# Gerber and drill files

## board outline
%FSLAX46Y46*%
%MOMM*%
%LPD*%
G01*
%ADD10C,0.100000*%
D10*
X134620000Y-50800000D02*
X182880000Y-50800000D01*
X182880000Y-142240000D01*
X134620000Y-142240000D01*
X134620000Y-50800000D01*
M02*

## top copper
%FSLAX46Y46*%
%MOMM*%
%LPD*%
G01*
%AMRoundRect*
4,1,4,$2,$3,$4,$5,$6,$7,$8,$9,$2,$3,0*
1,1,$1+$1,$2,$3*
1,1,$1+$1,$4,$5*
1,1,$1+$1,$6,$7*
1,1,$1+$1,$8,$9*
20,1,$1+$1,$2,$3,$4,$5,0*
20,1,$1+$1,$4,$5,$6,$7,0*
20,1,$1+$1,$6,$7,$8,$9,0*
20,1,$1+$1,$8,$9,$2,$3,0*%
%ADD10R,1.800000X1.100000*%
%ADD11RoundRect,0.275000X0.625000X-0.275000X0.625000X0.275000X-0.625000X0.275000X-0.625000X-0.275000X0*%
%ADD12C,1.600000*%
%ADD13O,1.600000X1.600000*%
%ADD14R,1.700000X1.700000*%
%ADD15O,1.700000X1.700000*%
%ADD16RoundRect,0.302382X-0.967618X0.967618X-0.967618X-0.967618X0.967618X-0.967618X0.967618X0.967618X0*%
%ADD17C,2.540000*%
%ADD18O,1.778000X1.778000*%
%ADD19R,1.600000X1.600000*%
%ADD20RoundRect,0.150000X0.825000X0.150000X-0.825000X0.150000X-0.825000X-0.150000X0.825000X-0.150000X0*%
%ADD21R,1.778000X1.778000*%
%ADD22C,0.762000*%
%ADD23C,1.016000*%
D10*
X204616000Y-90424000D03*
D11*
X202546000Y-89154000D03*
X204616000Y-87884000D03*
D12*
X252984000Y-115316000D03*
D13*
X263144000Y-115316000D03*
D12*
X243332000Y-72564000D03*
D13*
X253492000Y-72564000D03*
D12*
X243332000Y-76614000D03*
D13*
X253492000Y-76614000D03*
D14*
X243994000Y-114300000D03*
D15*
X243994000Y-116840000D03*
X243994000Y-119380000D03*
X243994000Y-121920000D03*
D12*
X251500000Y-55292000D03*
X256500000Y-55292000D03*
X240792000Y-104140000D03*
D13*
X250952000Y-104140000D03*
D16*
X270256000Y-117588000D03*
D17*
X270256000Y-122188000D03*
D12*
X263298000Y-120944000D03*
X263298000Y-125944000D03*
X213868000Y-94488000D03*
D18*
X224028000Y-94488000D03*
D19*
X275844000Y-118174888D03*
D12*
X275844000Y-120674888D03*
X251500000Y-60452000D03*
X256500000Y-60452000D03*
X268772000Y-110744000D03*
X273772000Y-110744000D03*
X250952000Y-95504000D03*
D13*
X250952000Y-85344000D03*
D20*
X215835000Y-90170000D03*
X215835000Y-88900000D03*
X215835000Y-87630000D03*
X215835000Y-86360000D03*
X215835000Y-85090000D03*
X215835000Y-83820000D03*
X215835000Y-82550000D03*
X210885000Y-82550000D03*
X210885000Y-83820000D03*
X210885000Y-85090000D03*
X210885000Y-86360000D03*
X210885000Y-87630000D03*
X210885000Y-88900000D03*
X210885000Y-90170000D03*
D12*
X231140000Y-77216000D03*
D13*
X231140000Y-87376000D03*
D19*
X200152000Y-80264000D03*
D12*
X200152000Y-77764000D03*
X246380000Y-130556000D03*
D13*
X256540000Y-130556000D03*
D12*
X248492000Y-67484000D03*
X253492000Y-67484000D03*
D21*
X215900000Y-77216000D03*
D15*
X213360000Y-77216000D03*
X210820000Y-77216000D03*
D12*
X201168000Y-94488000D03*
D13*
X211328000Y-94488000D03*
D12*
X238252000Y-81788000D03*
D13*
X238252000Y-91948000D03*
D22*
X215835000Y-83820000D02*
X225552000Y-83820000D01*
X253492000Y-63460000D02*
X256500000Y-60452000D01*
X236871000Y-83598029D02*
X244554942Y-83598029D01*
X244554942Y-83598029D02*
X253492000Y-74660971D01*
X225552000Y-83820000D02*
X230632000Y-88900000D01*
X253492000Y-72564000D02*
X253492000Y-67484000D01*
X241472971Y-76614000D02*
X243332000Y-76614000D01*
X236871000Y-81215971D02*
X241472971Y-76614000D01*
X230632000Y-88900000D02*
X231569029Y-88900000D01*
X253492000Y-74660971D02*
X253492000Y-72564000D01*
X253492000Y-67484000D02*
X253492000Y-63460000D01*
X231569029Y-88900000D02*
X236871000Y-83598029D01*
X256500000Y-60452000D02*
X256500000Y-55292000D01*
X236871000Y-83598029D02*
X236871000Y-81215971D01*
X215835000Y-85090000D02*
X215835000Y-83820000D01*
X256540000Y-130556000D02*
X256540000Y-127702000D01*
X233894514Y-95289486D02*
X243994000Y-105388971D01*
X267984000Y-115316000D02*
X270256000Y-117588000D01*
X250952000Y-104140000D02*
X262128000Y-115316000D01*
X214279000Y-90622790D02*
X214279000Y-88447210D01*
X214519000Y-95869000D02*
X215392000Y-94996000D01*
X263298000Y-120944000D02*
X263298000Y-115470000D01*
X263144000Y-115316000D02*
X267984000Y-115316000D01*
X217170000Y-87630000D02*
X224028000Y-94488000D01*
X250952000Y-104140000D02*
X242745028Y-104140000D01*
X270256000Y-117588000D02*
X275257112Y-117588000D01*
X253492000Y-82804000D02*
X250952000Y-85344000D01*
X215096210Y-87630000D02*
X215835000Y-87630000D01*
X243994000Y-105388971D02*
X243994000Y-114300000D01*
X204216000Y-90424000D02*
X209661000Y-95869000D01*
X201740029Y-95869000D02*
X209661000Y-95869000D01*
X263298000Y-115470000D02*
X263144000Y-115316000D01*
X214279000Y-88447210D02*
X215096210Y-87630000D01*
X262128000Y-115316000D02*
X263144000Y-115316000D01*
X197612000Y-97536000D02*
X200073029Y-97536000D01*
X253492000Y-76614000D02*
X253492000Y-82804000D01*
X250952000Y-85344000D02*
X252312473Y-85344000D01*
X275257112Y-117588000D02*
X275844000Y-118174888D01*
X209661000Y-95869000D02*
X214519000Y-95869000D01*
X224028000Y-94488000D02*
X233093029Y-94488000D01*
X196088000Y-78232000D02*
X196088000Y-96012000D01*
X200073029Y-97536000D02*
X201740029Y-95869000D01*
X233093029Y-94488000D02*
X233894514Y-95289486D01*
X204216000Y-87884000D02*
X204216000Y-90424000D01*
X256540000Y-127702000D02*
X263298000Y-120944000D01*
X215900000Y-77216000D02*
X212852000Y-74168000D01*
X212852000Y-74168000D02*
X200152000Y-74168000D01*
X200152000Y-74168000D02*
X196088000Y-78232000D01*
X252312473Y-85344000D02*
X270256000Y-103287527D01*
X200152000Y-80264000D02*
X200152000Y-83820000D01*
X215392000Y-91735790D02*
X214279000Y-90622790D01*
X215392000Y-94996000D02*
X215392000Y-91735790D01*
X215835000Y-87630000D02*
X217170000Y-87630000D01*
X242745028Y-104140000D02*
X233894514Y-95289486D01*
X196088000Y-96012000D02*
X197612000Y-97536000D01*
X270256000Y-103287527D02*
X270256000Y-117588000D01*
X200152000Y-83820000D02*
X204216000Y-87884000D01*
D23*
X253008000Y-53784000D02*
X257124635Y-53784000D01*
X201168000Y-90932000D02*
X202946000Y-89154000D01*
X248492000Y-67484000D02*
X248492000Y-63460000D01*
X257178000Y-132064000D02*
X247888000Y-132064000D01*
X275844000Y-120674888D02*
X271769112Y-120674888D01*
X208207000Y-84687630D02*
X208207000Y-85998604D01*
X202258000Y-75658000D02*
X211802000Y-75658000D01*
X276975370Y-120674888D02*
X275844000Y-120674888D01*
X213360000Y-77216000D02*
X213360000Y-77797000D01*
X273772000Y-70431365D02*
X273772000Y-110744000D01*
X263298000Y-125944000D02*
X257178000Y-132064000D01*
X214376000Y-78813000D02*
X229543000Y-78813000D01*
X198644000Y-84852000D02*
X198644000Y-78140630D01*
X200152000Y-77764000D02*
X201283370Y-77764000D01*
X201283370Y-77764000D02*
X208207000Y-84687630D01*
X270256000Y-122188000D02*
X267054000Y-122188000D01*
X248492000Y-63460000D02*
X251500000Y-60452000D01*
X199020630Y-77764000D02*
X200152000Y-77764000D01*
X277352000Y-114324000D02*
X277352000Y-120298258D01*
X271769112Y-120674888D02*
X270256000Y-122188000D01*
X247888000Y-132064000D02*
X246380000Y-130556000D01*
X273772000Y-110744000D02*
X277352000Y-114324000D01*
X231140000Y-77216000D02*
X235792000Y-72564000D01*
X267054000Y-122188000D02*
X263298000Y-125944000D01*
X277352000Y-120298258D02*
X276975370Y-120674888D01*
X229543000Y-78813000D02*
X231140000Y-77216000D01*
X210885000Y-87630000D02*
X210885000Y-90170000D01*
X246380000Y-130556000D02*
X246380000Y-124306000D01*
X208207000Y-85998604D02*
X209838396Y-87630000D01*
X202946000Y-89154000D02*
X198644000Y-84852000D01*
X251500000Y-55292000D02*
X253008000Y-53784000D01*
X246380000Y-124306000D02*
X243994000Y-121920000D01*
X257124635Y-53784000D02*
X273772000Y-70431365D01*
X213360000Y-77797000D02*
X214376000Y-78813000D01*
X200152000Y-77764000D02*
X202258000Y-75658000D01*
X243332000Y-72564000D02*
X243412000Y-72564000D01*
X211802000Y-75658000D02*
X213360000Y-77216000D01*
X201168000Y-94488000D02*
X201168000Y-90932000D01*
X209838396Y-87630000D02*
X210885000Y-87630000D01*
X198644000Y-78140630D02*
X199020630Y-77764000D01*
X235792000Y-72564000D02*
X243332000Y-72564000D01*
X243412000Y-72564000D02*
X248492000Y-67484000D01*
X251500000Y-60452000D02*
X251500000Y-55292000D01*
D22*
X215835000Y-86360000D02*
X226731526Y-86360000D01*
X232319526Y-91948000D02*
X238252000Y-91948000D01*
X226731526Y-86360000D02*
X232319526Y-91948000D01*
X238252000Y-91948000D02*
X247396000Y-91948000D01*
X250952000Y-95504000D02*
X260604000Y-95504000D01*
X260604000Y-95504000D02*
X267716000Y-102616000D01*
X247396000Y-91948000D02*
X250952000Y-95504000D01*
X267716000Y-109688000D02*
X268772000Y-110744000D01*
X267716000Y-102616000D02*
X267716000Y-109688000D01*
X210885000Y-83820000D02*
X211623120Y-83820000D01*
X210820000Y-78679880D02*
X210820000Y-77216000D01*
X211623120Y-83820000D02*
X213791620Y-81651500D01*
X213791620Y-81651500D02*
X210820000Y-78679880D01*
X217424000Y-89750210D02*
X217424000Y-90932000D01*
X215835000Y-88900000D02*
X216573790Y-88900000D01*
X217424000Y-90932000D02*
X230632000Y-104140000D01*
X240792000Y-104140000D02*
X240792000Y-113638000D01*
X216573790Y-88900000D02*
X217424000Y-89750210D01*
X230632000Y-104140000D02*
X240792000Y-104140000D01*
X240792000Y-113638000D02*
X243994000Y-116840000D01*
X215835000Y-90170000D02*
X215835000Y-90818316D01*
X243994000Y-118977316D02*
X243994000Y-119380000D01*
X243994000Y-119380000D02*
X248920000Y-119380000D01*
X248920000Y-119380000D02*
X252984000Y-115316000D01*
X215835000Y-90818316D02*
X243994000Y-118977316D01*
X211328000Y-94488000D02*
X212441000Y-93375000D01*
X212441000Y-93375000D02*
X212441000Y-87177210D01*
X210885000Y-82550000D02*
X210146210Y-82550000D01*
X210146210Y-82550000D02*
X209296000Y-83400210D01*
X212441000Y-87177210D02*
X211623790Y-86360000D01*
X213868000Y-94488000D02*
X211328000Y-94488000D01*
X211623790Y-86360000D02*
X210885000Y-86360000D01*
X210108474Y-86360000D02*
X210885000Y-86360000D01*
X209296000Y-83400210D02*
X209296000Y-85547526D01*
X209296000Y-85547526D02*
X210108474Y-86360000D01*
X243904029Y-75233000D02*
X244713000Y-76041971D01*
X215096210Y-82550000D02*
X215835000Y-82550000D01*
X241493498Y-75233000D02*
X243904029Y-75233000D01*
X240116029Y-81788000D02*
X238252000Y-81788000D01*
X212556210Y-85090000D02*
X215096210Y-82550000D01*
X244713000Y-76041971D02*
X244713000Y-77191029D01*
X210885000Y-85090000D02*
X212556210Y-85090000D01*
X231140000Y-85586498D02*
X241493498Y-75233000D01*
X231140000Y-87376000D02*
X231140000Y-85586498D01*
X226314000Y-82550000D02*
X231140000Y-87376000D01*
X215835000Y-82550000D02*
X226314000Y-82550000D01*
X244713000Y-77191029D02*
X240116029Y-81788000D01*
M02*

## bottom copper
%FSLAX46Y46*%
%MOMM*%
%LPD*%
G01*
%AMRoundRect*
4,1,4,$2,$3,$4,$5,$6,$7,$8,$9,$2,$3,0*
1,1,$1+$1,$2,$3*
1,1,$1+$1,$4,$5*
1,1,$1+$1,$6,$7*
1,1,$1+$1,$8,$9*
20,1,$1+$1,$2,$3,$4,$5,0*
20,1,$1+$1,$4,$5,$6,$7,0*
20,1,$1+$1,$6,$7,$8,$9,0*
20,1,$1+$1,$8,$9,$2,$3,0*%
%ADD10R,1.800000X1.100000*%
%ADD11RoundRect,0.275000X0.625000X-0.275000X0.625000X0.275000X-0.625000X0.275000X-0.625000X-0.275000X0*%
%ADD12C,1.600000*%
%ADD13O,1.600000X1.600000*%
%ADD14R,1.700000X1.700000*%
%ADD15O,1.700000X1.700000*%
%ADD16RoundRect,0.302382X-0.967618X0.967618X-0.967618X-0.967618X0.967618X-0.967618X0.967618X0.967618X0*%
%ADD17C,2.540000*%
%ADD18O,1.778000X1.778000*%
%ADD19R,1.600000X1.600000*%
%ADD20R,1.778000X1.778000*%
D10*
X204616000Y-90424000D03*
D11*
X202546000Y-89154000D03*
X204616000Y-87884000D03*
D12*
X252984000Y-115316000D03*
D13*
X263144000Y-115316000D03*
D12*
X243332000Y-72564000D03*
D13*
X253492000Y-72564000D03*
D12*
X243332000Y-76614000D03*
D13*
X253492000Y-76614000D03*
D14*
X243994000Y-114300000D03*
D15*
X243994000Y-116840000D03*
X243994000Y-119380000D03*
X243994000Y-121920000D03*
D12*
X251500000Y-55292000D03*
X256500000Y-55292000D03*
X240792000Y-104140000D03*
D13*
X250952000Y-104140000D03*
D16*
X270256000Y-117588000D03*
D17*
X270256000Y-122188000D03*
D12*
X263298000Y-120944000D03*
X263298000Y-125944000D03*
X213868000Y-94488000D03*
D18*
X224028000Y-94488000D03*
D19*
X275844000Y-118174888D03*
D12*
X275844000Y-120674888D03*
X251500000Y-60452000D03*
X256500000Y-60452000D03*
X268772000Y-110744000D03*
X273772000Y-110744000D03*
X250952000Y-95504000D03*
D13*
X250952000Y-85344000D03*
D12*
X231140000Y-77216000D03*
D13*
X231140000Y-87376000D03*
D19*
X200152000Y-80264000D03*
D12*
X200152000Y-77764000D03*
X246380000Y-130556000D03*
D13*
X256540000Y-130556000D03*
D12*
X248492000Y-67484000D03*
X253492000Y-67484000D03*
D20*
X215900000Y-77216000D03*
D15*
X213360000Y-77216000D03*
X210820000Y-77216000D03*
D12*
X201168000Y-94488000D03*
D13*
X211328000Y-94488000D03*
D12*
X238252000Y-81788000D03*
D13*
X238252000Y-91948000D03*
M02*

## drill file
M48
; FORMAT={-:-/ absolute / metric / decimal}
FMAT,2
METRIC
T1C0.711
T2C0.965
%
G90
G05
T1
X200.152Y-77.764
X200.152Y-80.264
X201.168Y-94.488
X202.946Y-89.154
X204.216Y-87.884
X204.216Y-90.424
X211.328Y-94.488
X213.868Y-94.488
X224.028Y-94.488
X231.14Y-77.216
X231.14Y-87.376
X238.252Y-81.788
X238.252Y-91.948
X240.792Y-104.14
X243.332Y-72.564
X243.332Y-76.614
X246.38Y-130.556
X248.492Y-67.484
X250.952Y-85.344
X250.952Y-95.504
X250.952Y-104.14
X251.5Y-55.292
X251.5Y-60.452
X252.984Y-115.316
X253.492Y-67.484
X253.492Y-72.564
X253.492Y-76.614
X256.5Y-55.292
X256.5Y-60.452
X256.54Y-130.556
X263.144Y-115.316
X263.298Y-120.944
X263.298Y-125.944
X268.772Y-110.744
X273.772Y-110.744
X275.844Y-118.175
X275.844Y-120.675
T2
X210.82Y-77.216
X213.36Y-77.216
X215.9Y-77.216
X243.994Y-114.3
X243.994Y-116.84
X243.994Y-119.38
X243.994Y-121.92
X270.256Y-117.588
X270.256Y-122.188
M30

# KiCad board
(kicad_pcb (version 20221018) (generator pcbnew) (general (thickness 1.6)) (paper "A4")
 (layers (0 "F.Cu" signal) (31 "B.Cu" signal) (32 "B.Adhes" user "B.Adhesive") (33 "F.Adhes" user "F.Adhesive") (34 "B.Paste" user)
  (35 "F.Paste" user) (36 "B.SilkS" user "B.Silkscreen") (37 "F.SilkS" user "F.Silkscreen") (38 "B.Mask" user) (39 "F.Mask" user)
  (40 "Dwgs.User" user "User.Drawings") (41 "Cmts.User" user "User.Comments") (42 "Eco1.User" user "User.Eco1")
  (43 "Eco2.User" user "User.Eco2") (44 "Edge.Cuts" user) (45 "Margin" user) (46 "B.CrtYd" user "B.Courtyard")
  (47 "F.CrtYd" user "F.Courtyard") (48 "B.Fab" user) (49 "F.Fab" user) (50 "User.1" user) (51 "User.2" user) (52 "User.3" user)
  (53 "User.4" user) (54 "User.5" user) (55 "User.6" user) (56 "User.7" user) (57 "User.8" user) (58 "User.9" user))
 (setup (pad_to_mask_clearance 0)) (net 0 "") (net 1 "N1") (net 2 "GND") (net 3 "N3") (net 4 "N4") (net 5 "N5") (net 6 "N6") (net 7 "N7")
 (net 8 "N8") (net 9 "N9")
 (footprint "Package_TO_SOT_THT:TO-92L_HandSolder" (layer "F.Cu") (at 204.216 90.424 90)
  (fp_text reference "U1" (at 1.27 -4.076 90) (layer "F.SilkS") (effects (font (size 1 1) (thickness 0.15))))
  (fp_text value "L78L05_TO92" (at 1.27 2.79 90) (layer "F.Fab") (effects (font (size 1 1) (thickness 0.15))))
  (pad "1" thru_hole rect (at 0 0 90) (size 1.1 1.8) (drill 0.7112 (offset 0 0.4)) (layers "*.Cu" "*.Mask") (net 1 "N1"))
  (pad "2" thru_hole roundrect (at 1.27 -1.27 90) (size 1.1 1.8) (drill 0.7112 (offset 0 -0.4)) (layers "*.Cu" "*.Mask")
   (roundrect_rratio 0.25) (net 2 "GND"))
  (pad "3" thru_hole roundrect (at 2.54 0 90) (size 1.1 1.8) (drill 0.7112 (offset 0 0.4)) (layers "*.Cu" "*.Mask") (roundrect_rratio 0.25)
   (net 1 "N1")))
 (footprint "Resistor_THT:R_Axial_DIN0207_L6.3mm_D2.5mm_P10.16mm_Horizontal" (layer "F.Cu") (at 252.984 115.316)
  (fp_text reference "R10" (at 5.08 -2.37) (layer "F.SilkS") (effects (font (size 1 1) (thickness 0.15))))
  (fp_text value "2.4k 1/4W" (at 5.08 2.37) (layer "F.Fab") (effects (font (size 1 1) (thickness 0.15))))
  (pad "1" thru_hole circle (at 0 0) (size 1.6 1.6) (drill 0.7112) (layers "*.Cu" "*.Mask") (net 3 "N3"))
  (pad "2" thru_hole oval (at 10.16 0) (size 1.6 1.6) (drill 0.7112) (layers "*.Cu" "*.Mask") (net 1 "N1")))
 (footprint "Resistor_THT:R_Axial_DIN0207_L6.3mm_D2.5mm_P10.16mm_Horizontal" (layer "F.Cu") (at 243.332 72.564)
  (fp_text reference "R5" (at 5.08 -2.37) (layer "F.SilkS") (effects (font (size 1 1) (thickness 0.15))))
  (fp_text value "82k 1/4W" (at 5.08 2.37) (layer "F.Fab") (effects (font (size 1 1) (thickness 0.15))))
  (pad "1" thru_hole circle (at 0 0) (size 1.6 1.6) (drill 0.7112) (layers "*.Cu" "*.Mask") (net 2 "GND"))
  (pad "2" thru_hole oval (at 10.16 0) (size 1.6 1.6) (drill 0.7112) (layers "*.Cu" "*.Mask") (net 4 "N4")))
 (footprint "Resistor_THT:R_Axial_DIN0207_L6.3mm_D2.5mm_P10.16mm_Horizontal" (layer "F.Cu") (at 243.332 76.614)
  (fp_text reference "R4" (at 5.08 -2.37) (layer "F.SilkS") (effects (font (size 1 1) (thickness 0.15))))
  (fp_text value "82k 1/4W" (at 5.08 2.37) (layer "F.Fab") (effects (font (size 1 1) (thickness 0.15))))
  (pad "1" thru_hole circle (at 0 0) (size 1.6 1.6) (drill 0.7112) (layers "*.Cu" "*.Mask") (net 4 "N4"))
  (pad "2" thru_hole oval (at 10.16 0) (size 1.6 1.6) (drill 0.7112) (layers "*.Cu" "*.Mask") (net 1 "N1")))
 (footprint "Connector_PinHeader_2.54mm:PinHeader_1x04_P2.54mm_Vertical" (layer "F.Cu") (at 243.994 114.3)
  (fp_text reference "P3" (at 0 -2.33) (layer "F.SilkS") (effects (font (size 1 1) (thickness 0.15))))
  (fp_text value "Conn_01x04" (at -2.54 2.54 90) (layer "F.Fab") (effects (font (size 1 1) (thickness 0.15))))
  (pad "1" thru_hole rect (at 0 0) (size 1.7 1.7) (drill 0.9652) (layers "*.Cu" "*.Mask") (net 1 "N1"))
  (pad "2" thru_hole oval (at 0 2.54) (size 1.7 1.7) (drill 0.9652) (layers "*.Cu" "*.Mask") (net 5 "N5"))
  (pad "3" thru_hole oval (at 0 5.08) (size 1.7 1.7) (drill 0.9652) (layers "*.Cu" "*.Mask") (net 3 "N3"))
  (pad "4" thru_hole oval (at 0 7.62) (size 1.7 1.7) (drill 0.9652) (layers "*.Cu" "*.Mask") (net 2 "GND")))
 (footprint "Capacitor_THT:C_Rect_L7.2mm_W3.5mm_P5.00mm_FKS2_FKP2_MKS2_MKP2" (layer "F.Cu") (at 251.5 55.292)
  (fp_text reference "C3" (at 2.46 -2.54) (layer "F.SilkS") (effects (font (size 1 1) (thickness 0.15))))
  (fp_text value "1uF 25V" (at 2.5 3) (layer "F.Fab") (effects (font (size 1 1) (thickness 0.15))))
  (pad "1" thru_hole circle (at 0 0) (size 1.6 1.6) (drill 0.7112) (layers "*.Cu" "*.Mask") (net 2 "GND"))
  (pad "2" thru_hole circle (at 5 0) (size 1.6 1.6) (drill 0.7112) (layers "*.Cu" "*.Mask") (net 4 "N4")))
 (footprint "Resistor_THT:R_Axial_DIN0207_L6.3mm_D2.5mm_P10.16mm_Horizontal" (layer "F.Cu") (at 240.792 104.14)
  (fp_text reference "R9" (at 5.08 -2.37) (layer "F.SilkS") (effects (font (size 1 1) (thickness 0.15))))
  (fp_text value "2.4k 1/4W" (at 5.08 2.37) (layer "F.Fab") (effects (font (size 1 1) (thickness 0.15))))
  (pad "1" thru_hole circle (at 0 0) (size 1.6 1.6) (drill 0.7112) (layers "*.Cu" "*.Mask") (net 5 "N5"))
  (pad "2" thru_hole oval (at 10.16 0) (size 1.6 1.6) (drill 0.7112) (layers "*.Cu" "*.Mask") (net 1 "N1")))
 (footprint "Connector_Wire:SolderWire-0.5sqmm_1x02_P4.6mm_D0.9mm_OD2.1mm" (layer "F.Cu") (at 270.256 117.588 -90)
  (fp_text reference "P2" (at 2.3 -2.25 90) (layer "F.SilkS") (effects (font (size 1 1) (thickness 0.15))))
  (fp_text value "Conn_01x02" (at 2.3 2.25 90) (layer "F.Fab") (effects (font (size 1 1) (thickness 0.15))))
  (pad "1" thru_hole roundrect (at 0 0 270) (size 2.54 2.54) (drill 0.9652) (layers "*.Cu" "*.Mask") (roundrect_rratio 0.119048)
   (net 1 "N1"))
  (pad "2" thru_hole circle (at 4.6 0 270) (size 2.54 2.54) (drill 0.9652) (layers "*.Cu" "*.Mask") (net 2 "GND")))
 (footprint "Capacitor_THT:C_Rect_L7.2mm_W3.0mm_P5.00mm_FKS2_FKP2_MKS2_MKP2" (layer "F.Cu") (at 263.298 120.944 -90)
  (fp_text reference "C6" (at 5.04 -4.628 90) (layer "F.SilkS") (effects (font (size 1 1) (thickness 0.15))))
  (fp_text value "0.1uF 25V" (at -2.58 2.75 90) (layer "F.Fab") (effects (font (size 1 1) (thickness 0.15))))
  (pad "1" thru_hole circle (at 0 0 270) (size 1.6 1.6) (drill 0.7112) (layers "*.Cu" "*.Mask") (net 1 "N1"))
  (pad "2" thru_hole circle (at 5 0 270) (size 1.6 1.6) (drill 0.7112) (layers "*.Cu" "*.Mask") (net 2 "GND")))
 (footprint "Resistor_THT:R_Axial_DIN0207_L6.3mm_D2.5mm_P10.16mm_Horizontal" (layer "F.Cu") (at 213.868 94.488)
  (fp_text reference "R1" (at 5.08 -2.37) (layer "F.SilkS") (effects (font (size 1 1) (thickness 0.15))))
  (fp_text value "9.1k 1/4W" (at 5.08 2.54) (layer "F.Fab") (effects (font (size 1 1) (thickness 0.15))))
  (pad "1" thru_hole circle (at 0 0) (size 1.6 1.6) (drill 0.7112) (layers "*.Cu" "*.Mask") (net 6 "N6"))
  (pad "2" thru_hole oval (at 10.16 0) (size 1.778 1.778) (drill 0.7112) (layers "*.Cu" "*.Mask") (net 1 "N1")))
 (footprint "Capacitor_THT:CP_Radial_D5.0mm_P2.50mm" (layer "F.Cu") (at 275.844 118.174888 -90)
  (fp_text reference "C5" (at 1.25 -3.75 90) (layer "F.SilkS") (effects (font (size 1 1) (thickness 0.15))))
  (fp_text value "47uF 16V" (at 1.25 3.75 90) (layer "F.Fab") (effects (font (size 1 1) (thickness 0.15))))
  (pad "1" thru_hole rect (at 0 0 270) (size 1.6 1.6) (drill 0.7112) (layers "*.Cu" "*.Mask") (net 1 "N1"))
  (pad "2" thru_hole circle (at 2.5 0 270) (size 1.6 1.6) (drill 0.7112) (layers "*.Cu" "*.Mask") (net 2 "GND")))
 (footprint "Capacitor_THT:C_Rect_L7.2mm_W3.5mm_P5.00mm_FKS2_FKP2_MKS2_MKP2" (layer "F.Cu") (at 251.5 60.452)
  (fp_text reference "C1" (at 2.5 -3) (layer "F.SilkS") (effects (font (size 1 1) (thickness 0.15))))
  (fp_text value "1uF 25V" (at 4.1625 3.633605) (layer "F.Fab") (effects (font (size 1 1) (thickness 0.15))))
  (pad "1" thru_hole circle (at 0 0) (size 1.6 1.6) (drill 0.7112) (layers "*.Cu" "*.Mask") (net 2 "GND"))
  (pad "2" thru_hole circle (at 5 0) (size 1.6 1.6) (drill 0.7112) (layers "*.Cu" "*.Mask") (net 4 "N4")))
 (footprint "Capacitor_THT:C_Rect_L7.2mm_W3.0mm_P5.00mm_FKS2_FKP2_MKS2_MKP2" (layer "F.Cu") (at 268.772 110.744)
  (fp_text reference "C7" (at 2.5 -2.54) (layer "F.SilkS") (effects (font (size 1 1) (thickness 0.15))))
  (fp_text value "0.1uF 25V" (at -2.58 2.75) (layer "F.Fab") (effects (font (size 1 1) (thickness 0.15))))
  (pad "1" thru_hole circle (at 0 0) (size 1.6 1.6) (drill 0.7112) (layers "*.Cu" "*.Mask") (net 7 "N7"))
  (pad "2" thru_hole circle (at 5 0) (size 1.6 1.6) (drill 0.7112) (layers "*.Cu" "*.Mask") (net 2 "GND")))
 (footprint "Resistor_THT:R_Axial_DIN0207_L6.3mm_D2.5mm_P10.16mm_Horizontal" (layer "F.Cu") (at 250.952 95.504 90)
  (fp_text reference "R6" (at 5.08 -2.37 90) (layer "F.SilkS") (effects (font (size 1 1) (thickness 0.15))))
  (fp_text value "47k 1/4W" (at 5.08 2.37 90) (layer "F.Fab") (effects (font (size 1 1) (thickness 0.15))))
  (pad "1" thru_hole circle (at 0 0 90) (size 1.6 1.6) (drill 0.7112) (layers "*.Cu" "*.Mask") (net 7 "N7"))
  (pad "2" thru_hole oval (at 10.16 0 90) (size 1.6 1.6) (drill 0.7112) (layers "*.Cu" "*.Mask") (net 1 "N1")))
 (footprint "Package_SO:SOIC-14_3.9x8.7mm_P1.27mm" (layer "F.Cu") (at 213.36 86.36 180)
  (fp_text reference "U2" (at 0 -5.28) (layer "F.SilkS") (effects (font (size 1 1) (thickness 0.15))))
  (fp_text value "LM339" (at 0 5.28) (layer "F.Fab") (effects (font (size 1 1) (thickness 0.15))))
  (pad "1" smd roundrect (at -2.475 -3.81 180) (size 1.95 0.6) (layers "F.Cu" "F.Paste" "F.Mask") (roundrect_rratio 0.25) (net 3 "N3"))
  (pad "2" smd roundrect (at -2.475 -2.54 180) (size 1.95 0.6) (layers "F.Cu" "F.Paste" "F.Mask") (roundrect_rratio 0.25) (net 5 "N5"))
  (pad "3" smd roundrect (at -2.475 -1.27 180) (size 1.95 0.6) (layers "F.Cu" "F.Paste" "F.Mask") (roundrect_rratio 0.25) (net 1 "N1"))
  (pad "4" smd roundrect (at -2.475 0 180) (size 1.95 0.6) (layers "F.Cu" "F.Paste" "F.Mask") (roundrect_rratio 0.25) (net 7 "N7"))
  (pad "5" smd roundrect (at -2.475 1.27 180) (size 1.95 0.6) (layers "F.Cu" "F.Paste" "F.Mask") (roundrect_rratio 0.25) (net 4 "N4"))
  (pad "6" smd roundrect (at -2.475 2.54 180) (size 1.95 0.6) (layers "F.Cu" "F.Paste" "F.Mask") (roundrect_rratio 0.25) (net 4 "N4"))
  (pad "7" smd roundrect (at -2.475 3.81 180) (size 1.95 0.6) (layers "F.Cu" "F.Paste" "F.Mask") (roundrect_rratio 0.25) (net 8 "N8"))
  (pad "8" smd roundrect (at 2.475 3.81 180) (size 1.95 0.6) (layers "F.Cu" "F.Paste" "F.Mask") (roundrect_rratio 0.25) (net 6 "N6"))
  (pad "9" smd roundrect (at 2.475 2.54 180) (size 1.95 0.6) (layers "F.Cu" "F.Paste" "F.Mask") (roundrect_rratio 0.25) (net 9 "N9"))
  (pad "10" smd roundrect (at 2.475 1.27 180) (size 1.95 0.6) (layers "F.Cu" "F.Paste" "F.Mask") (roundrect_rratio 0.25) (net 8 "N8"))
  (pad "11" smd roundrect (at 2.475 0 180) (size 1.95 0.6) (layers "F.Cu" "F.Paste" "F.Mask") (roundrect_rratio 0.25) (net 6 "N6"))
  (pad "12" smd roundrect (at 2.475 -1.27 180) (size 1.95 0.6) (layers "F.Cu" "F.Paste" "F.Mask") (roundrect_rratio 0.25) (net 2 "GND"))
  (pad "13" smd roundrect (at 2.475 -2.54 180) (size 1.95 0.6) (layers "F.Cu" "F.Paste" "F.Mask") (roundrect_rratio 0.25) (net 2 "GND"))
  (pad "14" smd roundrect (at 2.475 -3.81 180) (size 1.95 0.6) (layers "F.Cu" "F.Paste" "F.Mask") (roundrect_rratio 0.25) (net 2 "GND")))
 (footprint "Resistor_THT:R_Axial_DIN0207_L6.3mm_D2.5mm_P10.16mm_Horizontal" (layer "F.Cu") (at 231.14 77.216 -90)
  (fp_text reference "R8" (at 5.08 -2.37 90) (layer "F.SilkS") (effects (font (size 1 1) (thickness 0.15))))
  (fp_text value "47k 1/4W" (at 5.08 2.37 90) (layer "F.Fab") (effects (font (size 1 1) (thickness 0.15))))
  (pad "1" thru_hole circle (at 0 0 270) (size 1.6 1.6) (drill 0.7112) (layers "*.Cu" "*.Mask") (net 2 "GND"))
  (pad "2" thru_hole oval (at 10.16 0 270) (size 1.6 1.6) (drill 0.7112) (layers "*.Cu" "*.Mask") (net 8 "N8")))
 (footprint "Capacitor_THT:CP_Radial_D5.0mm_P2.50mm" (layer "F.Cu") (at 200.152 80.264 90)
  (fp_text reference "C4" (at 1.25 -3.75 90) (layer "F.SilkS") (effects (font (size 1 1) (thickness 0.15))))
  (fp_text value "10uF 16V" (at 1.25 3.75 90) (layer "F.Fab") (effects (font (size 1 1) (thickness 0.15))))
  (pad "1" thru_hole rect (at 0 0 90) (size 1.6 1.6) (drill 0.7112) (layers "*.Cu" "*.Mask") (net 1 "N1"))
  (pad "2" thru_hole circle (at 2.5 0 90) (size 1.6 1.6) (drill 0.7112) (layers "*.Cu" "*.Mask") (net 2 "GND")))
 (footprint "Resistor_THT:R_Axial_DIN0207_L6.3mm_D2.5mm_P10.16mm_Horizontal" (layer "F.Cu") (at 246.38 130.556)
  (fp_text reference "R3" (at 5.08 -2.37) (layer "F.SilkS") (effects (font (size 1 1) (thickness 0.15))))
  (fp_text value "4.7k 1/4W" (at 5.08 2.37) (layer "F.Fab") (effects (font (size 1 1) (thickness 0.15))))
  (pad "1" thru_hole circle (at 0 0) (size 1.6 1.6) (drill 0.7112) (layers "*.Cu" "*.Mask") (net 2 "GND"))
  (pad "2" thru_hole oval (at 10.16 0) (size 1.6 1.6) (drill 0.7112) (layers "*.Cu" "*.Mask") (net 1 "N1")))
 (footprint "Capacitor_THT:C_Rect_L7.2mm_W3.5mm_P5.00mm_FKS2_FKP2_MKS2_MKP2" (layer "F.Cu") (at 248.492 67.484)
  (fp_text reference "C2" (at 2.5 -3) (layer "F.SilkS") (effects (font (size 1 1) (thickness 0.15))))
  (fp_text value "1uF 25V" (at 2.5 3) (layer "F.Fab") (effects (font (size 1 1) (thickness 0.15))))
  (pad "1" thru_hole circle (at 0 0) (size 1.6 1.6) (drill 0.7112) (layers "*.Cu" "*.Mask") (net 2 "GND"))
  (pad "2" thru_hole circle (at 5 0) (size 1.6 1.6) (drill 0.7112) (layers "*.Cu" "*.Mask") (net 4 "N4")))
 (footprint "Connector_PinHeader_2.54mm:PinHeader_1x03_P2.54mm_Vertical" (layer "F.Cu") (at 215.9 77.216 -90)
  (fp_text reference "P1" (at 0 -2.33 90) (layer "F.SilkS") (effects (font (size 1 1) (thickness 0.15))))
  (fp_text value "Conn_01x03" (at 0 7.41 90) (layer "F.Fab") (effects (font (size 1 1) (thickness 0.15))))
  (pad "1" thru_hole rect (at 0 0 270) (size 1.778 1.778) (drill 0.9652) (layers "*.Cu" "*.Mask") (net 1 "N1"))
  (pad "2" thru_hole oval (at 0 2.54 270) (size 1.7 1.7) (drill 0.9652) (layers "*.Cu" "*.Mask") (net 2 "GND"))
  (pad "3" thru_hole oval (at 0 5.08 270) (size 1.7 1.7) (drill 0.9652) (layers "*.Cu" "*.Mask") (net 9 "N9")))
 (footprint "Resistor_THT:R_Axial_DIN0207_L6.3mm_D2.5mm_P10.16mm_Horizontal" (layer "F.Cu") (at 201.168 94.488)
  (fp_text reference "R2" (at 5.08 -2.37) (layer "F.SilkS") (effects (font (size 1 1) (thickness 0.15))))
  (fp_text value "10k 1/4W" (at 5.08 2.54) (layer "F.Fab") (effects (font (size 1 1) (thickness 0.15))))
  (pad "1" thru_hole circle (at 0 0) (size 1.6 1.6) (drill 0.7112) (layers "*.Cu" "*.Mask") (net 2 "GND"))
  (pad "2" thru_hole oval (at 10.16 0) (size 1.6 1.6) (drill 0.7112) (layers "*.Cu" "*.Mask") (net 6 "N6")))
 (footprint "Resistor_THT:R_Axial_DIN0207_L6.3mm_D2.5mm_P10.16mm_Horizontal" (layer "F.Cu") (at 238.252 81.788 -90)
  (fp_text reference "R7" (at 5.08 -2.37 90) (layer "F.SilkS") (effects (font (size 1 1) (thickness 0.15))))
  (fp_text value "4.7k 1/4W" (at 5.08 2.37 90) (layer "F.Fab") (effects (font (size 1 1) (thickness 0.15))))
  (pad "1" thru_hole circle (at 0 0 270) (size 1.6 1.6) (drill 0.7112) (layers "*.Cu" "*.Mask") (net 8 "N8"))
  (pad "2" thru_hole oval (at 10.16 0 270) (size 1.6 1.6) (drill 0.7112) (layers "*.Cu" "*.Mask") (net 7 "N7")))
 (gr_rect (start 134.62 50.8) (end 182.88 142.24) (stroke (width 0.1) (type default)) (fill none) (layer "Edge.Cuts"))
 (segment (start 215.835 83.82) (end 225.552 83.82) (width 0.762) (layer "F.Cu") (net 4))
 (segment (start 253.492 63.46) (end 256.5 60.452) (width 0.762) (layer "F.Cu") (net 4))
 (segment (start 236.871 83.598029) (end 244.554942 83.598029) (width 0.762) (layer "F.Cu") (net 4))
 (segment (start 244.554942 83.598029) (end 253.492 74.660971) (width 0.762) (layer "F.Cu") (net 4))
 (segment (start 225.552 83.82) (end 230.632 88.9) (width 0.762) (layer "F.Cu") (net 4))
 (segment (start 253.492 72.564) (end 253.492 67.484) (width 0.762) (layer "F.Cu") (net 4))
 (segment (start 241.472971 76.614) (end 243.332 76.614) (width 0.762) (layer "F.Cu") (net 4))
 (segment (start 236.871 81.215971) (end 241.472971 76.614) (width 0.762) (layer "F.Cu") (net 4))
 (segment (start 230.632 88.9) (end 231.569029 88.9) (width 0.762) (layer "F.Cu") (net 4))
 (segment (start 253.492 74.660971) (end 253.492 72.564) (width 0.762) (layer "F.Cu") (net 4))
 (segment (start 253.492 67.484) (end 253.492 63.46) (width 0.762) (layer "F.Cu") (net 4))
 (segment (start 231.569029 88.9) (end 236.871 83.598029) (width 0.762) (layer "F.Cu") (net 4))
 (segment (start 256.5 60.452) (end 256.5 55.292) (width 0.762) (layer "F.Cu") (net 4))
 (segment (start 236.871 83.598029) (end 236.871 81.215971) (width 0.762) (layer "F.Cu") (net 4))
 (segment (start 215.835 85.09) (end 215.835 83.82) (width 0.762) (layer "F.Cu") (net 4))
 (segment (start 256.54 130.556) (end 256.54 127.702) (width 0.762) (layer "F.Cu") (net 1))
 (segment (start 233.894514 95.289486) (end 243.994 105.388971) (width 0.762) (layer "F.Cu") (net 1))
 (segment (start 267.984 115.316) (end 270.256 117.588) (width 0.762) (layer "F.Cu") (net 1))
 (segment (start 250.952 104.14) (end 262.128 115.316) (width 0.762) (layer "F.Cu") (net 1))
 (segment (start 214.279 90.62279) (end 214.279 88.44721) (width 0.762) (layer "F.Cu") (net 1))
 (segment (start 214.519 95.869) (end 215.392 94.996) (width 0.762) (layer "F.Cu") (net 1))
 (segment (start 263.298 120.944) (end 263.298 115.47) (width 0.762) (layer "F.Cu") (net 1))
 (segment (start 263.144 115.316) (end 267.984 115.316) (width 0.762) (layer "F.Cu") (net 1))
 (segment (start 217.17 87.63) (end 224.028 94.488) (width 0.762) (layer "F.Cu") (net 1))
 (segment (start 250.952 104.14) (end 242.745028 104.14) (width 0.762) (layer "F.Cu") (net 1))
 (segment (start 270.256 117.588) (end 275.257112 117.588) (width 0.762) (layer "F.Cu") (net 1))
 (segment (start 253.492 82.804) (end 250.952 85.344) (width 0.762) (layer "F.Cu") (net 1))
 (segment (start 215.09621 87.63) (end 215.835 87.63) (width 0.762) (layer "F.Cu") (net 1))
 (segment (start 243.994 105.388971) (end 243.994 114.3) (width 0.762) (layer "F.Cu") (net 1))
 (segment (start 204.216 90.424) (end 209.661 95.869) (width 0.762) (layer "F.Cu") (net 1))
 (segment (start 201.740029 95.869) (end 209.661 95.869) (width 0.762) (layer "F.Cu") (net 1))
 (segment (start 263.298 115.47) (end 263.144 115.316) (width 0.762) (layer "F.Cu") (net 1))
 (segment (start 214.279 88.44721) (end 215.09621 87.63) (width 0.762) (layer "F.Cu") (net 1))
 (segment (start 262.128 115.316) (end 263.144 115.316) (width 0.762) (layer "F.Cu") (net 1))
 (segment (start 197.612 97.536) (end 200.073029 97.536) (width 0.762) (layer "F.Cu") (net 1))
 (segment (start 253.492 76.614) (end 253.492 82.804) (width 0.762) (layer "F.Cu") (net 1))
 (segment (start 250.952 85.344) (end 252.312473 85.344) (width 0.762) (layer "F.Cu") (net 1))
 (segment (start 275.257112 117.588) (end 275.844 118.174888) (width 0.762) (layer "F.Cu") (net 1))
 (segment (start 209.661 95.869) (end 214.519 95.869) (width 0.762) (layer "F.Cu") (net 1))
 (segment (start 224.028 94.488) (end 233.093029 94.488) (width 0.762) (layer "F.Cu") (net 1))
 (segment (start 196.088 78.232) (end 196.088 96.012) (width 0.762) (layer "F.Cu") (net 1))
 (segment (start 200.073029 97.536) (end 201.740029 95.869) (width 0.762) (layer "F.Cu") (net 1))
 (segment (start 233.093029 94.488) (end 233.894514 95.289486) (width 0.762) (layer "F.Cu") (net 1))
 (segment (start 204.216 87.884) (end 204.216 90.424) (width 0.762) (layer "F.Cu") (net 1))
 (segment (start 256.54 127.702) (end 263.298 120.944) (width 0.762) (layer "F.Cu") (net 1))
 (segment (start 215.9 77.216) (end 212.852 74.168) (width 0.762) (layer "F.Cu") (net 1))
 (segment (start 212.852 74.168) (end 200.152 74.168) (width 0.762) (layer "F.Cu") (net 1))
 (segment (start 200.152 74.168) (end 196.088 78.232) (width 0.762) (layer "F.Cu") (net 1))
 (segment (start 252.312473 85.344) (end 270.256 103.287527) (width 0.762) (layer "F.Cu") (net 1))
 (segment (start 200.152 80.264) (end 200.152 83.82) (width 0.762) (layer "F.Cu") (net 1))
 (segment (start 215.392 91.73579) (end 214.279 90.62279) (width 0.762) (layer "F.Cu") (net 1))
 (segment (start 215.392 94.996) (end 215.392 91.73579) (width 0.762) (layer "F.Cu") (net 1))
 (segment (start 215.835 87.63) (end 217.17 87.63) (width 0.762) (layer "F.Cu") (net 1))
 (segment (start 242.745028 104.14) (end 233.894514 95.289486) (width 0.762) (layer "F.Cu") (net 1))
 (segment (start 196.088 96.012) (end 197.612 97.536) (width 0.762) (layer "F.Cu") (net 1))
 (segment (start 270.256 103.287527) (end 270.256 117.588) (width 0.762) (layer "F.Cu") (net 1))
 (segment (start 200.152 83.82) (end 204.216 87.884) (width 0.762) (layer "F.Cu") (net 1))
 (segment (start 253.008 53.784) (end 257.124635 53.784) (width 1.016) (layer "F.Cu") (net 2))
 (segment (start 201.168 90.932) (end 202.946 89.154) (width 1.016) (layer "F.Cu") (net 2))
 (segment (start 248.492 67.484) (end 248.492 63.46) (width 1.016) (layer "F.Cu") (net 2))
 (segment (start 257.178 132.064) (end 247.888 132.064) (width 1.016) (layer "F.Cu") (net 2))
 (segment (start 275.844 120.674888) (end 271.769112 120.674888) (width 1.016) (layer "F.Cu") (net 2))
 (segment (start 208.207 84.68763) (end 208.207 85.998604) (width 1.016) (layer "F.Cu") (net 2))
 (segment (start 202.258 75.658) (end 211.802 75.658) (width 1.016) (layer "F.Cu") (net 2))
 (segment (start 276.97537 120.674888) (end 275.844 120.674888) (width 1.016) (layer "F.Cu") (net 2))
 (segment (start 213.36 77.216) (end 213.36 77.797) (width 1.016) (layer "F.Cu") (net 2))
 (segment (start 273.772 70.431365) (end 273.772 110.744) (width 1.016) (layer "F.Cu") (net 2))
 (segment (start 263.298 125.944) (end 257.178 132.064) (width 1.016) (layer "F.Cu") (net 2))
 (segment (start 214.376 78.813) (end 229.543 78.813) (width 1.016) (layer "F.Cu") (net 2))
 (segment (start 198.644 84.852) (end 198.644 78.14063) (width 1.016) (layer "F.Cu") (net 2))
 (segment (start 200.152 77.764) (end 201.28337 77.764) (width 1.016) (layer "F.Cu") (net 2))
 (segment (start 201.28337 77.764) (end 208.207 84.68763) (width 1.016) (layer "F.Cu") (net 2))
 (segment (start 270.256 122.188) (end 267.054 122.188) (width 1.016) (layer "F.Cu") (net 2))
 (segment (start 248.492 63.46) (end 251.5 60.452) (width 1.016) (layer "F.Cu") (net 2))
 (segment (start 199.02063 77.764) (end 200.152 77.764) (width 1.016) (layer "F.Cu") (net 2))
 (segment (start 277.352 114.324) (end 277.352 120.298258) (width 1.016) (layer "F.Cu") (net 2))
 (segment (start 271.769112 120.674888) (end 270.256 122.188) (width 1.016) (layer "F.Cu") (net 2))
 (segment (start 247.888 132.064) (end 246.38 130.556) (width 1.016) (layer "F.Cu") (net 2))
 (segment (start 273.772 110.744) (end 277.352 114.324) (width 1.016) (layer "F.Cu") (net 2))
 (segment (start 231.14 77.216) (end 235.792 72.564) (width 1.016) (layer "F.Cu") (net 2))
 (segment (start 267.054 122.188) (end 263.298 125.944) (width 1.016) (layer "F.Cu") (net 2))
 (segment (start 277.352 120.298258) (end 276.97537 120.674888) (width 1.016) (layer "F.Cu") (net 2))
 (segment (start 229.543 78.813) (end 231.14 77.216) (width 1.016) (layer "F.Cu") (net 2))
 (segment (start 210.885 87.63) (end 210.885 90.17) (width 1.016) (layer "F.Cu") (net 2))
 (segment (start 246.38 130.556) (end 246.38 124.306) (width 1.016) (layer "F.Cu") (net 2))
 (segment (start 208.207 85.998604) (end 209.838396 87.63) (width 1.016) (layer "F.Cu") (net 2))
 (segment (start 202.946 89.154) (end 198.644 84.852) (width 1.016) (layer "F.Cu") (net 2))
 (segment (start 251.5 55.292) (end 253.008 53.784) (width 1.016) (layer "F.Cu") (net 2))
 (segment (start 246.38 124.306) (end 243.994 121.92) (width 1.016) (layer "F.Cu") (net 2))
 (segment (start 257.124635 53.784) (end 273.772 70.431365) (width 1.016) (layer "F.Cu") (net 2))
 (segment (start 213.36 77.797) (end 214.376 78.813) (width 1.016) (layer "F.Cu") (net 2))
 (segment (start 200.152 77.764) (end 202.258 75.658) (width 1.016) (layer "F.Cu") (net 2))
 (segment (start 243.332 72.564) (end 243.412 72.564) (width 1.016) (layer "F.Cu") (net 2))
 (segment (start 211.802 75.658) (end 213.36 77.216) (width 1.016) (layer "F.Cu") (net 2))
 (segment (start 201.168 94.488) (end 201.168 90.932) (width 1.016) (layer "F.Cu") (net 2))
 (segment (start 209.838396 87.63) (end 210.885 87.63) (width 1.016) (layer "F.Cu") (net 2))
 (segment (start 198.644 78.14063) (end 199.02063 77.764) (width 1.016) (layer "F.Cu") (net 2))
 (segment (start 235.792 72.564) (end 243.332 72.564) (width 1.016) (layer "F.Cu") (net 2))
 (segment (start 243.412 72.564) (end 248.492 67.484) (width 1.016) (layer "F.Cu") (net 2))
 (segment (start 251.5 60.452) (end 251.5 55.292) (width 1.016) (layer "F.Cu") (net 2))
 (segment (start 215.835 86.36) (end 226.731526 86.36) (width 0.762) (layer "F.Cu") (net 7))
 (segment (start 232.319526 91.948) (end 238.252 91.948) (width 0.762) (layer "F.Cu") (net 7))
 (segment (start 226.731526 86.36) (end 232.319526 91.948) (width 0.762) (layer "F.Cu") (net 7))
 (segment (start 238.252 91.948) (end 247.396 91.948) (width 0.762) (layer "F.Cu") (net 7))
 (segment (start 250.952 95.504) (end 260.604 95.504) (width 0.762) (layer "F.Cu") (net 7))
 (segment (start 260.604 95.504) (end 267.716 102.616) (width 0.762) (layer "F.Cu") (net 7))
 (segment (start 247.396 91.948) (end 250.952 95.504) (width 0.762) (layer "F.Cu") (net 7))
 (segment (start 267.716 109.688) (end 268.772 110.744) (width 0.762) (layer "F.Cu") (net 7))
 (segment (start 267.716 102.616) (end 267.716 109.688) (width 0.762) (layer "F.Cu") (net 7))
 (segment (start 210.885 83.82) (end 211.62312 83.82) (width 0.762) (layer "F.Cu") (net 9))
 (segment (start 210.82 78.67988) (end 210.82 77.216) (width 0.762) (layer "F.Cu") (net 9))
 (segment (start 211.62312 83.82) (end 213.79162 81.6515) (width 0.762) (layer "F.Cu") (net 9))
 (segment (start 213.79162 81.6515) (end 210.82 78.67988) (width 0.762) (layer "F.Cu") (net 9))
 (segment (start 217.424 89.75021) (end 217.424 90.932) (width 0.762) (layer "F.Cu") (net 5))
 (segment (start 215.835 88.9) (end 216.57379 88.9) (width 0.762) (layer "F.Cu") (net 5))
 (segment (start 217.424 90.932) (end 230.632 104.14) (width 0.762) (layer "F.Cu") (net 5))
 (segment (start 240.792 104.14) (end 240.792 113.638) (width 0.762) (layer "F.Cu") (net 5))
 (segment (start 216.57379 88.9) (end 217.424 89.75021) (width 0.762) (layer "F.Cu") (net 5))
 (segment (start 230.632 104.14) (end 240.792 104.14) (width 0.762) (layer "F.Cu") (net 5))
 (segment (start 240.792 113.638) (end 243.994 116.84) (width 0.762) (layer "F.Cu") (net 5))
 (segment (start 215.835 90.17) (end 215.835 90.818316) (width 0.762) (layer "F.Cu") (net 3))
 (segment (start 243.994 118.977316) (end 243.994 119.38) (width 0.762) (layer "F.Cu") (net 3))
 (segment (start 243.994 119.38) (end 248.92 119.38) (width 0.762) (layer "F.Cu") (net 3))
 (segment (start 248.92 119.38) (end 252.984 115.316) (width 0.762) (layer "F.Cu") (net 3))
 (segment (start 215.835 90.818316) (end 243.994 118.977316) (width 0.762) (layer "F.Cu") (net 3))
 (segment (start 211.328 94.488) (end 212.441 93.375) (width 0.762) (layer "F.Cu") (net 6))
 (segment (start 212.441 93.375) (end 212.441 87.17721) (width 0.762) (layer "F.Cu") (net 6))
 (segment (start 210.885 82.55) (end 210.14621 82.55) (width 0.762) (layer "F.Cu") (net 6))
 (segment (start 210.14621 82.55) (end 209.296 83.40021) (width 0.762) (layer "F.Cu") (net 6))
 (segment (start 212.441 87.17721) (end 211.62379 86.36) (width 0.762) (layer "F.Cu") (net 6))
 (segment (start 213.868 94.488) (end 211.328 94.488) (width 0.762) (layer "F.Cu") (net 6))
 (segment (start 211.62379 86.36) (end 210.885 86.36) (width 0.762) (layer "F.Cu") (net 6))
 (segment (start 210.108474 86.36) (end 210.885 86.36) (width 0.762) (layer "F.Cu") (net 6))
 (segment (start 209.296 83.40021) (end 209.296 85.547526) (width 0.762) (layer "F.Cu") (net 6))
 (segment (start 209.296 85.547526) (end 210.108474 86.36) (width 0.762) (layer "F.Cu") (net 6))
 (segment (start 243.904029 75.233) (end 244.713 76.041971) (width 0.762) (layer "F.Cu") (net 8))
 (segment (start 215.09621 82.55) (end 215.835 82.55) (width 0.762) (layer "F.Cu") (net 8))
 (segment (start 241.493498 75.233) (end 243.904029 75.233) (width 0.762) (layer "F.Cu") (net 8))
 (segment (start 240.116029 81.788) (end 238.252 81.788) (width 0.762) (layer "F.Cu") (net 8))
 (segment (start 212.55621 85.09) (end 215.09621 82.55) (width 0.762) (layer "F.Cu") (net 8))
 (segment (start 244.713 76.041971) (end 244.713 77.191029) (width 0.762) (layer "F.Cu") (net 8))
 (segment (start 210.885 85.09) (end 212.55621 85.09) (width 0.762) (layer "F.Cu") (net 8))
 (segment (start 231.14 85.586498) (end 241.493498 75.233) (width 0.762) (layer "F.Cu") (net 8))
 (segment (start 231.14 87.376) (end 231.14 85.586498) (width 0.762) (layer "F.Cu") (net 8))
 (segment (start 226.314 82.55) (end 231.14 87.376) (width 0.762) (layer "F.Cu") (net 8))
 (segment (start 215.835 82.55) (end 226.314 82.55) (width 0.762) (layer "F.Cu") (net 8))
 (segment (start 244.713 77.191029) (end 240.116029 81.788) (width 0.762) (layer "F.Cu") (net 8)))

